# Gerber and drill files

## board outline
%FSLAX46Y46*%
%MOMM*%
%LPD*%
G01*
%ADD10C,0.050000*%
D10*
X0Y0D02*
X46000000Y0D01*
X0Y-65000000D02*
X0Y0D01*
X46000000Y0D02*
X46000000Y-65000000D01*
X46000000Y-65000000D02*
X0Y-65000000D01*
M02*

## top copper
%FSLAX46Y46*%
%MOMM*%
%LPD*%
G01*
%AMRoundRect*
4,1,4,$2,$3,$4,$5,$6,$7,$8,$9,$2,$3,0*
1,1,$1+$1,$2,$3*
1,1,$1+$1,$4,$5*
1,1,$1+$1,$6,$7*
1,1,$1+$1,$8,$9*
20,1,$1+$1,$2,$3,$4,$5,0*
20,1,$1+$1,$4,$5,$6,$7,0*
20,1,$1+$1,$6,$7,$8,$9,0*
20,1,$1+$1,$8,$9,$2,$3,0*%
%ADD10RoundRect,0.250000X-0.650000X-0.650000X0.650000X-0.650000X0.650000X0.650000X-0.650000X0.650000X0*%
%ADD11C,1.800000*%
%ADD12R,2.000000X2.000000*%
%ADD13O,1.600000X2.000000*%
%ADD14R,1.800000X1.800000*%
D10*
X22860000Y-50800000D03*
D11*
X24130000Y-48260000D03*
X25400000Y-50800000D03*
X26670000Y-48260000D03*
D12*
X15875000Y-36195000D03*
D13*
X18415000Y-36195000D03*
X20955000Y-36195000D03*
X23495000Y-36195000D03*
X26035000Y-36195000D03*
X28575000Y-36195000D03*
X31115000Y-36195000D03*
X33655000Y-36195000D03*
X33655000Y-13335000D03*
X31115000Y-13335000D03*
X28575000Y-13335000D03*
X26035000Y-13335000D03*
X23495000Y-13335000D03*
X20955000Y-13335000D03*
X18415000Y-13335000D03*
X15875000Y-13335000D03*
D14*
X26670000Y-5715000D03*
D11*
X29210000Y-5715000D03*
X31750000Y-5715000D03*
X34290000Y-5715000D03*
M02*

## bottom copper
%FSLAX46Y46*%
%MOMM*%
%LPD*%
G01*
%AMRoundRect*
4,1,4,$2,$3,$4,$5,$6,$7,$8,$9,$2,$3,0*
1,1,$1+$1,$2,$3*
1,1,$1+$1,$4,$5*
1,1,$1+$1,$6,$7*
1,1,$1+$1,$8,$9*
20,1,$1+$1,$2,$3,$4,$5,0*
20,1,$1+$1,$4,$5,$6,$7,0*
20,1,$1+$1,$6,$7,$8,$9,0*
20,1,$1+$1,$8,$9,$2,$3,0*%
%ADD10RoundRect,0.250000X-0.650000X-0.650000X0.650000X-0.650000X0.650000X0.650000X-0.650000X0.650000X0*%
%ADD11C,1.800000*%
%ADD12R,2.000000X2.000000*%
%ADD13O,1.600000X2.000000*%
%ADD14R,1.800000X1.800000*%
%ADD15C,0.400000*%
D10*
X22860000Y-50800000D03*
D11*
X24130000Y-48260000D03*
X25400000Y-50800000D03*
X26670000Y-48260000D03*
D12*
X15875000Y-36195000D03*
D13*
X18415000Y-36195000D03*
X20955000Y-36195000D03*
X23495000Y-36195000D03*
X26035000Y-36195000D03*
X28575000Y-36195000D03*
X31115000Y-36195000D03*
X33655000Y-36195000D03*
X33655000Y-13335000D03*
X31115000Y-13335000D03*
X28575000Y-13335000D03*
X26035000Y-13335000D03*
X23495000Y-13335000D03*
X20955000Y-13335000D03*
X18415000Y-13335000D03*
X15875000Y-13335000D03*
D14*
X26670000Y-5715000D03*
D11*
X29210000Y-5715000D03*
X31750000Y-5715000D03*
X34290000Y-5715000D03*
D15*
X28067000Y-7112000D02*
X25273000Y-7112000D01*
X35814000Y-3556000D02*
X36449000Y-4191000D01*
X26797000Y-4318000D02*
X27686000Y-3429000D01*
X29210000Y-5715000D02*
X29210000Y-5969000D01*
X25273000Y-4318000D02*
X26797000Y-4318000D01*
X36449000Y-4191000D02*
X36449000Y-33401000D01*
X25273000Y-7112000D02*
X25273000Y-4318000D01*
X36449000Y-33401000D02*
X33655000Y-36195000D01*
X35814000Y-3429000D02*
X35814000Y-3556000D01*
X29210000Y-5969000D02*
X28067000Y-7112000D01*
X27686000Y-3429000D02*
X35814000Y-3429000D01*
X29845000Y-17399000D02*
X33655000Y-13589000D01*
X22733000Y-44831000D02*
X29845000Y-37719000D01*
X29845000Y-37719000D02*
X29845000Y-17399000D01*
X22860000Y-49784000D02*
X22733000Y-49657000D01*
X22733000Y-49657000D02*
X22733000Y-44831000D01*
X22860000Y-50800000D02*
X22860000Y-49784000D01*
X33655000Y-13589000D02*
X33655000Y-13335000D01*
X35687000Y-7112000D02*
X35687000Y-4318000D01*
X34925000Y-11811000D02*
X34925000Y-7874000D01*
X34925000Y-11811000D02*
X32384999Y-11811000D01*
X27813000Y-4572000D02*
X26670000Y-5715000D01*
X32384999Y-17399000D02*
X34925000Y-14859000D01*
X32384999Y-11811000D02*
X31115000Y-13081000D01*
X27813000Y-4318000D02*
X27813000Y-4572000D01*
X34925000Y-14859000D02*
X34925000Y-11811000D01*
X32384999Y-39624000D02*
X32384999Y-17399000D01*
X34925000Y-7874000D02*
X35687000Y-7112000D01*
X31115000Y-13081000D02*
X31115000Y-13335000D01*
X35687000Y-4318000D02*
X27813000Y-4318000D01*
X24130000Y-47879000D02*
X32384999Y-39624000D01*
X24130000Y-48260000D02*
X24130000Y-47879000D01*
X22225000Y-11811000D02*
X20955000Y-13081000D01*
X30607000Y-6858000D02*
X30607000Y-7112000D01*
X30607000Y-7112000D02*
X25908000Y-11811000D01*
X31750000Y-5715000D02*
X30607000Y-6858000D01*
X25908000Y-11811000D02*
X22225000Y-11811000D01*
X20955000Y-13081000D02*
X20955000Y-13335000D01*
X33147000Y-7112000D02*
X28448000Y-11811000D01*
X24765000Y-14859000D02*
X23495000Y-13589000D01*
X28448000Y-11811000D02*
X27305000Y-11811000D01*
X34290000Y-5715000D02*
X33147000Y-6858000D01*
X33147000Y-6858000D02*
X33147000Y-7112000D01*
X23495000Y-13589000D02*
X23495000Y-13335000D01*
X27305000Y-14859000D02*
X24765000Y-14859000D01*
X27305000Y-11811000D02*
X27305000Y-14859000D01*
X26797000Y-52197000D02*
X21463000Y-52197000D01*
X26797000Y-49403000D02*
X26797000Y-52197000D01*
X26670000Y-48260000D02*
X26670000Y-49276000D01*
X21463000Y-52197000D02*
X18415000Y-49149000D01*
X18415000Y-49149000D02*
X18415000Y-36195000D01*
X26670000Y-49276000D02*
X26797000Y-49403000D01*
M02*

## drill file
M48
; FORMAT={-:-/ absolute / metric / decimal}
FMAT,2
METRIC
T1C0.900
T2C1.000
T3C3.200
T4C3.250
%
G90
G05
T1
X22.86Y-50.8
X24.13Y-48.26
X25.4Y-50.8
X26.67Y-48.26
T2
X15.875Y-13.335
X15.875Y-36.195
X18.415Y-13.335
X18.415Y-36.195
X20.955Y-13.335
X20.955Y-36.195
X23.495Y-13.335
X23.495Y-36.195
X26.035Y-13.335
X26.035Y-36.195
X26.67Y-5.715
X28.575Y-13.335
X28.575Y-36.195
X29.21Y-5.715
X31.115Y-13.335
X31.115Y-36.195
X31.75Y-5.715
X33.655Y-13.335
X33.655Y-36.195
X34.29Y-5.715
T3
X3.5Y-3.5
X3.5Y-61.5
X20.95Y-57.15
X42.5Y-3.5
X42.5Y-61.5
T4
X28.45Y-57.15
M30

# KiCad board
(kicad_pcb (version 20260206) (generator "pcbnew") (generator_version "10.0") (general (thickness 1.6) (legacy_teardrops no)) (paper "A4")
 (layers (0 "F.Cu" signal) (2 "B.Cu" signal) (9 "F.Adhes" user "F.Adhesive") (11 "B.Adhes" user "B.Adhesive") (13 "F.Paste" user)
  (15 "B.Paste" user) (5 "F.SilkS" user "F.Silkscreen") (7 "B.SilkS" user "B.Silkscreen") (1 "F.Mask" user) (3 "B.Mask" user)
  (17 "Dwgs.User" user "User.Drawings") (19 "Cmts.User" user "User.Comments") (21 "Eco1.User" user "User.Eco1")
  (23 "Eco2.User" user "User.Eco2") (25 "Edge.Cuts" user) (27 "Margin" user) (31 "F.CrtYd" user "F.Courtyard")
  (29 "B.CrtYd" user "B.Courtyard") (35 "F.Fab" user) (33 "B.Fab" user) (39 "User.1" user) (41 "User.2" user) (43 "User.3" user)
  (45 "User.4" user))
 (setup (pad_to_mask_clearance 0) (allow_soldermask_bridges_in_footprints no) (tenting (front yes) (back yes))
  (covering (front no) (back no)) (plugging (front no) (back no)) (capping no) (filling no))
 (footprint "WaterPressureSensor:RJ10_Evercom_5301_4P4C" (layer "F.Cu") (at 22.86 50.8)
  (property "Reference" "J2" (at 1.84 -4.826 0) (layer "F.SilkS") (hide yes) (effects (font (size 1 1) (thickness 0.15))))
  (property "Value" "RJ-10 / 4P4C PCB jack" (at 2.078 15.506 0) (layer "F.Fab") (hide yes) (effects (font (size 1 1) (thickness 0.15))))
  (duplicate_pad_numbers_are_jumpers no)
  (pad "" np_thru_hole circle (at -1.91 6.35) (size 3.25 3.25) (drill 3.2) (layers "*.Mask"))
  (pad "" np_thru_hole circle (at 5.59 6.35) (size 3.25 3.25) (drill 3.25) (layers "*.Mask"))
  (pad "1" thru_hole roundrect (at 0 0) (size 1.8 1.8) (drill 0.9) (layers "*.Cu") (remove_unused_layers no) (roundrect_rratio 0.1388888889)
   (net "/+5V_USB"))
  (pad "2" thru_hole circle (at 1.27 -2.54) (size 1.8 1.8) (drill 0.9) (layers "*.Cu") (remove_unused_layers no) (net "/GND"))
  (pad "3" thru_hole circle (at 2.54 0) (size 1.8 1.8) (drill 0.9) (layers "*.Cu") (remove_unused_layers no) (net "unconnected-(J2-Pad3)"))
  (pad "4" thru_hole circle (at 3.81 -2.54) (size 1.8 1.8) (drill 0.9) (layers "*.Cu") (remove_unused_layers no) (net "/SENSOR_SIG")))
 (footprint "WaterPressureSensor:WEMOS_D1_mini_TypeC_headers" (layer "F.Cu") (at 15.875 36.195 90)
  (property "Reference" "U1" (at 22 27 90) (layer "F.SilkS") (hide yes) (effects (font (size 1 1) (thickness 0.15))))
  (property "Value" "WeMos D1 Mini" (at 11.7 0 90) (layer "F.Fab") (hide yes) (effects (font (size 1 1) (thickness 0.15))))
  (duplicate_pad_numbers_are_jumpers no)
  (pad "1" thru_hole rect (at 0 0 90) (size 2 2) (drill 1) (layers "*.Cu") (remove_unused_layers no) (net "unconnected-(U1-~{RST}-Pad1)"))
  (pad "2" thru_hole oval (at 0 2.54 90) (size 2 1.6) (drill 1) (layers "*.Cu") (remove_unused_layers no) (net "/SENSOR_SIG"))
  (pad "3" thru_hole oval (at 0 5.08 90) (size 2 1.6) (drill 1) (layers "*.Cu") (remove_unused_layers no) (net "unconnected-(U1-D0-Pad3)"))
  (pad "4" thru_hole oval (at 0 7.62 90) (size 2 1.6) (drill 1) (layers "*.Cu") (remove_unused_layers no)
   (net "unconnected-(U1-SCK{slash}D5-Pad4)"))
  (pad "5" thru_hole oval (at 0 10.16 90) (size 2 1.6) (drill 1) (layers "*.Cu") (remove_unused_layers no)
   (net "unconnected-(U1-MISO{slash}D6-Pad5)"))
  (pad "6" thru_hole oval (at 0 12.7 90) (size 2 1.6) (drill 1) (layers "*.Cu") (remove_unused_layers no)
   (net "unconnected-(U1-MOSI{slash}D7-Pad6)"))
  (pad "7" thru_hole oval (at 0 15.24 90) (size 2 1.6) (drill 1) (layers "*.Cu") (remove_unused_layers no)
   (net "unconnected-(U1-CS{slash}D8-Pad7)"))
  (pad "8" thru_hole oval (at 0 17.78 90) (size 2 1.6) (drill 1) (layers "*.Cu") (remove_unused_layers no) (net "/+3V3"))
  (pad "9" thru_hole oval (at 22.86 17.78 90) (size 2 1.6) (drill 1) (layers "*.Cu") (remove_unused_layers no) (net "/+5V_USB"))
  (pad "10" thru_hole oval (at 22.86 15.24 90) (size 2 1.6) (drill 1) (layers "*.Cu") (remove_unused_layers no) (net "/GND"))
  (pad "11" thru_hole oval (at 22.86 12.7 90) (size 2 1.6) (drill 1) (layers "*.Cu") (remove_unused_layers no)
   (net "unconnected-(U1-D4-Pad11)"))
  (pad "12" thru_hole oval (at 22.86 10.16 90) (size 2 1.6) (drill 1) (layers "*.Cu") (remove_unused_layers no)
   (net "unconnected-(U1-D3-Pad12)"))
  (pad "13" thru_hole oval (at 22.86 7.62 90) (size 2 1.6) (drill 1) (layers "*.Cu") (remove_unused_layers no) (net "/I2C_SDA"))
  (pad "14" thru_hole oval (at 22.86 5.08 90) (size 2 1.6) (drill 1) (layers "*.Cu") (remove_unused_layers no) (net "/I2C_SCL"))
  (pad "15" thru_hole oval (at 22.86 2.54 90) (size 2 1.6) (drill 1) (layers "*.Cu") (remove_unused_layers no)
   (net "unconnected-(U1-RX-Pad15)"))
  (pad "16" thru_hole oval (at 22.86 0 90) (size 2 1.6) (drill 1) (layers "*.Cu") (remove_unused_layers no)
   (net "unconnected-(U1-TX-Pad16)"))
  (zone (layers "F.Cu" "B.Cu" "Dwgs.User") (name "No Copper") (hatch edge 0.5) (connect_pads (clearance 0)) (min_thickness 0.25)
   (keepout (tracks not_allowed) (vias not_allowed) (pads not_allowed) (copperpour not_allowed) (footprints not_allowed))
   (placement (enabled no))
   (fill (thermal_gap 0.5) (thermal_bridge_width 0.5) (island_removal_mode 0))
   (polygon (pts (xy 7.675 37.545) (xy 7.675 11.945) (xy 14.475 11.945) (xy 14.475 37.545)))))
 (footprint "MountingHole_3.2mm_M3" (layer "F.Cu") (at 42.5 3.5)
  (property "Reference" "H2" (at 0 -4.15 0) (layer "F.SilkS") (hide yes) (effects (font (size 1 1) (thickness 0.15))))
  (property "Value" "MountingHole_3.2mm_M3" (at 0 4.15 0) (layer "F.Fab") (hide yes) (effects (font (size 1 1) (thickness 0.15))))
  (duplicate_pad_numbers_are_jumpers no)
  (pad "" np_thru_hole circle (at 0 0) (size 3.2 3.2) (drill 3.2) (layers "*.Cu" "F.Mask")))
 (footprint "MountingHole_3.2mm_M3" (layer "F.Cu") (at 42.5 61.5)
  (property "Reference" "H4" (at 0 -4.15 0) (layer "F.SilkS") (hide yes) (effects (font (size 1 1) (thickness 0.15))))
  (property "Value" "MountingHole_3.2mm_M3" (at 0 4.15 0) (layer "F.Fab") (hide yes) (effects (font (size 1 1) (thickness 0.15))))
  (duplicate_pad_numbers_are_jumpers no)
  (pad "" np_thru_hole circle (at 0 0) (size 3.2 3.2) (drill 3.2) (layers "*.Cu" "F.Mask")))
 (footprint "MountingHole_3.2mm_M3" (layer "F.Cu") (at 3.5 3.5)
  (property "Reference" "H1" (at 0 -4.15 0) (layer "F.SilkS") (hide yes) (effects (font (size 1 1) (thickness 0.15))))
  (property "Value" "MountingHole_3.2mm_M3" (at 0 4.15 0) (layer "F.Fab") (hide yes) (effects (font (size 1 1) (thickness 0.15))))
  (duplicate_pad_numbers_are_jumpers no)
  (pad "" np_thru_hole circle (at 0 0) (size 3.2 3.2) (drill 3.2) (layers "*.Cu" "F.Mask")))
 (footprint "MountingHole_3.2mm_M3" (layer "F.Cu") (at 3.5 61.5)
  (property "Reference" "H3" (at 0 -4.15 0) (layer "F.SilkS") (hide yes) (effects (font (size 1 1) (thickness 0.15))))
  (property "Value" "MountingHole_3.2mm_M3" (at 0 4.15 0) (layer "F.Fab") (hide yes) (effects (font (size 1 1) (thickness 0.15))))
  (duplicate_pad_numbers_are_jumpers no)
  (pad "" np_thru_hole circle (at 0 0) (size 3.2 3.2) (drill 3.2) (layers "*.Cu" "F.Mask")))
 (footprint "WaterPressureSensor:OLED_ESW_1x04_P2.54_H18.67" (layer "F.Cu") (at 26.67 5.715 90)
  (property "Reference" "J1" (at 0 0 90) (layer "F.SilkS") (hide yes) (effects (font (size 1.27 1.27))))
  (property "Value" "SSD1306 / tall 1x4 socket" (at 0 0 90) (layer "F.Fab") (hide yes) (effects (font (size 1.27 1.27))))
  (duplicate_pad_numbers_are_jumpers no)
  (pad "1" thru_hole rect (at 0 0 90) (size 1.8 1.8) (drill 1) (layers "*.Cu") (remove_unused_layers no) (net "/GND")
   (thermal_bridge_angle 45))
  (pad "2" thru_hole circle (at 0 2.54 90) (size 1.8 1.8) (drill 1) (layers "*.Cu") (remove_unused_layers no) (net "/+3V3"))
  (pad "3" thru_hole circle (at 0 5.08 90) (size 1.8 1.8) (drill 1) (layers "*.Cu") (remove_unused_layers no) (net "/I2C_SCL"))
  (pad "4" thru_hole circle (at 0 7.62 90) (size 1.8 1.8) (drill 1) (layers "*.Cu") (remove_unused_layers no) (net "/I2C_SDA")))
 (gr_line (start 0 0) (end 46 0) (stroke (width 0.05) (type default)) (layer "Edge.Cuts"))
 (gr_line (start 0 65) (end 0 0) (stroke (width 0.05) (type default)) (layer "Edge.Cuts"))
 (gr_line (start 46 0) (end 46 65) (stroke (width 0.05) (type default)) (layer "Edge.Cuts"))
 (gr_line (start 46 65) (end 0 65) (stroke (width 0.05) (type default)) (layer "Edge.Cuts"))
 (segment (start 28.067 7.112) (end 25.273 7.112) (width 0.4) (layer "B.Cu") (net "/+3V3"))
 (segment (start 35.814 3.556) (end 36.449 4.191) (width 0.4) (layer "B.Cu") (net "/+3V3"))
 (segment (start 26.797 4.318) (end 27.686 3.429) (width 0.4) (layer "B.Cu") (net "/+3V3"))
 (segment (start 29.21 5.715) (end 29.21 5.969) (width 0.4) (layer "B.Cu") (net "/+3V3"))
 (segment (start 25.273 4.318) (end 26.797 4.318) (width 0.4) (layer "B.Cu") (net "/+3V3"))
 (segment (start 36.449 4.191) (end 36.449 33.401) (width 0.4) (layer "B.Cu") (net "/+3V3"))
 (segment (start 25.273 7.112) (end 25.273 4.318) (width 0.4) (layer "B.Cu") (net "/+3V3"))
 (segment (start 36.449 33.401) (end 33.655 36.195) (width 0.4) (layer "B.Cu") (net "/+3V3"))
 (segment (start 35.814 3.429) (end 35.814 3.556) (width 0.4) (layer "B.Cu") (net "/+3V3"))
 (segment (start 29.21 5.969) (end 28.067 7.112) (width 0.4) (layer "B.Cu") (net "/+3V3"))
 (segment (start 27.686 3.429) (end 35.814 3.429) (width 0.4) (layer "B.Cu") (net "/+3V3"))
 (segment (start 29.845 17.399) (end 33.655 13.589) (width 0.4) (layer "B.Cu") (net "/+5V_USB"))
 (segment (start 22.733 44.831) (end 29.845 37.719) (width 0.4) (layer "B.Cu") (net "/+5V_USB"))
 (segment (start 29.845 37.719) (end 29.845 17.399) (width 0.4) (layer "B.Cu") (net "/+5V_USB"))
 (segment (start 22.86 49.784) (end 22.733 49.657) (width 0.4) (layer "B.Cu") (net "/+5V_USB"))
 (segment (start 22.733 49.657) (end 22.733 44.831) (width 0.4) (layer "B.Cu") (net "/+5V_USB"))
 (segment (start 22.86 50.8) (end 22.86 49.784) (width 0.4) (layer "B.Cu") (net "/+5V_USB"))
 (segment (start 33.655 13.589) (end 33.655 13.335) (width 0.4) (layer "B.Cu") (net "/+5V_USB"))
 (segment (start 35.687 7.112) (end 35.687 4.318) (width 0.4) (layer "B.Cu") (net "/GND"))
 (segment (start 34.925 11.811) (end 34.925 7.874) (width 0.4) (layer "B.Cu") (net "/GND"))
 (segment (start 34.925 11.811) (end 32.384999 11.811) (width 0.4) (layer "B.Cu") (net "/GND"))
 (segment (start 27.813 4.572) (end 26.67 5.715) (width 0.4) (layer "B.Cu") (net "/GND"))
 (segment (start 32.384999 17.399) (end 34.925 14.859) (width 0.4) (layer "B.Cu") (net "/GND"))
 (segment (start 32.384999 11.811) (end 31.115 13.081) (width 0.4) (layer "B.Cu") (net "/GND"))
 (segment (start 27.813 4.318) (end 27.813 4.572) (width 0.4) (layer "B.Cu") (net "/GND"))
 (segment (start 34.925 14.859) (end 34.925 11.811) (width 0.4) (layer "B.Cu") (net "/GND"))
 (segment (start 32.384999 39.624) (end 32.384999 17.399) (width 0.4) (layer "B.Cu") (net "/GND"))
 (segment (start 34.925 7.874) (end 35.687 7.112) (width 0.4) (layer "B.Cu") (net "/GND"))
 (segment (start 31.115 13.081) (end 31.115 13.335) (width 0.4) (layer "B.Cu") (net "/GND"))
 (segment (start 35.687 4.318) (end 27.813 4.318) (width 0.4) (layer "B.Cu") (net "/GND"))
 (segment (start 24.13 47.879) (end 32.384999 39.624) (width 0.4) (layer "B.Cu") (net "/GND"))
 (segment (start 24.13 48.26) (end 24.13 47.879) (width 0.4) (layer "B.Cu") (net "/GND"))
 (segment (start 22.225 11.811) (end 20.955 13.081) (width 0.4) (layer "B.Cu") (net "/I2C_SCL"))
 (segment (start 30.607 6.858) (end 30.607 7.112) (width 0.4) (layer "B.Cu") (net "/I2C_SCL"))
 (segment (start 30.607 7.112) (end 25.908 11.811) (width 0.4) (layer "B.Cu") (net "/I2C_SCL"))
 (segment (start 31.75 5.715) (end 30.607 6.858) (width 0.4) (layer "B.Cu") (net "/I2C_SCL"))
 (segment (start 25.908 11.811) (end 22.225 11.811) (width 0.4) (layer "B.Cu") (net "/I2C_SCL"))
 (segment (start 20.955 13.081) (end 20.955 13.335) (width 0.4) (layer "B.Cu") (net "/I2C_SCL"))
 (segment (start 33.147 7.112) (end 28.448 11.811) (width 0.4) (layer "B.Cu") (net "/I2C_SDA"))
 (segment (start 24.765 14.859) (end 23.495 13.589) (width 0.4) (layer "B.Cu") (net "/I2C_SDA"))
 (segment (start 28.448 11.811) (end 27.305 11.811) (width 0.4) (layer "B.Cu") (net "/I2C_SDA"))
 (segment (start 34.29 5.715) (end 33.147 6.858) (width 0.4) (layer "B.Cu") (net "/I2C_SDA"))
 (segment (start 33.147 6.858) (end 33.147 7.112) (width 0.4) (layer "B.Cu") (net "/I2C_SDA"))
 (segment (start 23.495 13.589) (end 23.495 13.335) (width 0.4) (layer "B.Cu") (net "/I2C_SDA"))
 (segment (start 27.305 14.859) (end 24.765 14.859) (width 0.4) (layer "B.Cu") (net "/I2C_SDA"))
 (segment (start 27.305 11.811) (end 27.305 14.859) (width 0.4) (layer "B.Cu") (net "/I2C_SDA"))
 (segment (start 26.797 52.197) (end 21.463 52.197) (width 0.4) (layer "B.Cu") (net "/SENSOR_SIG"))
 (segment (start 26.797 49.403) (end 26.797 52.197) (width 0.4) (layer "B.Cu") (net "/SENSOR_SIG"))
 (segment (start 26.67 48.26) (end 26.67 49.276) (width 0.4) (layer "B.Cu") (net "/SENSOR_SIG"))
 (segment (start 21.463 52.197) (end 18.415 49.149) (width 0.4) (layer "B.Cu") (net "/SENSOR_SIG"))
 (segment (start 18.415 49.149) (end 18.415 36.195) (width 0.4) (layer "B.Cu") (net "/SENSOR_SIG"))
 (segment (start 26.67 49.276) (end 26.797 49.403) (width 0.4) (layer "B.Cu") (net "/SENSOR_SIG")))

